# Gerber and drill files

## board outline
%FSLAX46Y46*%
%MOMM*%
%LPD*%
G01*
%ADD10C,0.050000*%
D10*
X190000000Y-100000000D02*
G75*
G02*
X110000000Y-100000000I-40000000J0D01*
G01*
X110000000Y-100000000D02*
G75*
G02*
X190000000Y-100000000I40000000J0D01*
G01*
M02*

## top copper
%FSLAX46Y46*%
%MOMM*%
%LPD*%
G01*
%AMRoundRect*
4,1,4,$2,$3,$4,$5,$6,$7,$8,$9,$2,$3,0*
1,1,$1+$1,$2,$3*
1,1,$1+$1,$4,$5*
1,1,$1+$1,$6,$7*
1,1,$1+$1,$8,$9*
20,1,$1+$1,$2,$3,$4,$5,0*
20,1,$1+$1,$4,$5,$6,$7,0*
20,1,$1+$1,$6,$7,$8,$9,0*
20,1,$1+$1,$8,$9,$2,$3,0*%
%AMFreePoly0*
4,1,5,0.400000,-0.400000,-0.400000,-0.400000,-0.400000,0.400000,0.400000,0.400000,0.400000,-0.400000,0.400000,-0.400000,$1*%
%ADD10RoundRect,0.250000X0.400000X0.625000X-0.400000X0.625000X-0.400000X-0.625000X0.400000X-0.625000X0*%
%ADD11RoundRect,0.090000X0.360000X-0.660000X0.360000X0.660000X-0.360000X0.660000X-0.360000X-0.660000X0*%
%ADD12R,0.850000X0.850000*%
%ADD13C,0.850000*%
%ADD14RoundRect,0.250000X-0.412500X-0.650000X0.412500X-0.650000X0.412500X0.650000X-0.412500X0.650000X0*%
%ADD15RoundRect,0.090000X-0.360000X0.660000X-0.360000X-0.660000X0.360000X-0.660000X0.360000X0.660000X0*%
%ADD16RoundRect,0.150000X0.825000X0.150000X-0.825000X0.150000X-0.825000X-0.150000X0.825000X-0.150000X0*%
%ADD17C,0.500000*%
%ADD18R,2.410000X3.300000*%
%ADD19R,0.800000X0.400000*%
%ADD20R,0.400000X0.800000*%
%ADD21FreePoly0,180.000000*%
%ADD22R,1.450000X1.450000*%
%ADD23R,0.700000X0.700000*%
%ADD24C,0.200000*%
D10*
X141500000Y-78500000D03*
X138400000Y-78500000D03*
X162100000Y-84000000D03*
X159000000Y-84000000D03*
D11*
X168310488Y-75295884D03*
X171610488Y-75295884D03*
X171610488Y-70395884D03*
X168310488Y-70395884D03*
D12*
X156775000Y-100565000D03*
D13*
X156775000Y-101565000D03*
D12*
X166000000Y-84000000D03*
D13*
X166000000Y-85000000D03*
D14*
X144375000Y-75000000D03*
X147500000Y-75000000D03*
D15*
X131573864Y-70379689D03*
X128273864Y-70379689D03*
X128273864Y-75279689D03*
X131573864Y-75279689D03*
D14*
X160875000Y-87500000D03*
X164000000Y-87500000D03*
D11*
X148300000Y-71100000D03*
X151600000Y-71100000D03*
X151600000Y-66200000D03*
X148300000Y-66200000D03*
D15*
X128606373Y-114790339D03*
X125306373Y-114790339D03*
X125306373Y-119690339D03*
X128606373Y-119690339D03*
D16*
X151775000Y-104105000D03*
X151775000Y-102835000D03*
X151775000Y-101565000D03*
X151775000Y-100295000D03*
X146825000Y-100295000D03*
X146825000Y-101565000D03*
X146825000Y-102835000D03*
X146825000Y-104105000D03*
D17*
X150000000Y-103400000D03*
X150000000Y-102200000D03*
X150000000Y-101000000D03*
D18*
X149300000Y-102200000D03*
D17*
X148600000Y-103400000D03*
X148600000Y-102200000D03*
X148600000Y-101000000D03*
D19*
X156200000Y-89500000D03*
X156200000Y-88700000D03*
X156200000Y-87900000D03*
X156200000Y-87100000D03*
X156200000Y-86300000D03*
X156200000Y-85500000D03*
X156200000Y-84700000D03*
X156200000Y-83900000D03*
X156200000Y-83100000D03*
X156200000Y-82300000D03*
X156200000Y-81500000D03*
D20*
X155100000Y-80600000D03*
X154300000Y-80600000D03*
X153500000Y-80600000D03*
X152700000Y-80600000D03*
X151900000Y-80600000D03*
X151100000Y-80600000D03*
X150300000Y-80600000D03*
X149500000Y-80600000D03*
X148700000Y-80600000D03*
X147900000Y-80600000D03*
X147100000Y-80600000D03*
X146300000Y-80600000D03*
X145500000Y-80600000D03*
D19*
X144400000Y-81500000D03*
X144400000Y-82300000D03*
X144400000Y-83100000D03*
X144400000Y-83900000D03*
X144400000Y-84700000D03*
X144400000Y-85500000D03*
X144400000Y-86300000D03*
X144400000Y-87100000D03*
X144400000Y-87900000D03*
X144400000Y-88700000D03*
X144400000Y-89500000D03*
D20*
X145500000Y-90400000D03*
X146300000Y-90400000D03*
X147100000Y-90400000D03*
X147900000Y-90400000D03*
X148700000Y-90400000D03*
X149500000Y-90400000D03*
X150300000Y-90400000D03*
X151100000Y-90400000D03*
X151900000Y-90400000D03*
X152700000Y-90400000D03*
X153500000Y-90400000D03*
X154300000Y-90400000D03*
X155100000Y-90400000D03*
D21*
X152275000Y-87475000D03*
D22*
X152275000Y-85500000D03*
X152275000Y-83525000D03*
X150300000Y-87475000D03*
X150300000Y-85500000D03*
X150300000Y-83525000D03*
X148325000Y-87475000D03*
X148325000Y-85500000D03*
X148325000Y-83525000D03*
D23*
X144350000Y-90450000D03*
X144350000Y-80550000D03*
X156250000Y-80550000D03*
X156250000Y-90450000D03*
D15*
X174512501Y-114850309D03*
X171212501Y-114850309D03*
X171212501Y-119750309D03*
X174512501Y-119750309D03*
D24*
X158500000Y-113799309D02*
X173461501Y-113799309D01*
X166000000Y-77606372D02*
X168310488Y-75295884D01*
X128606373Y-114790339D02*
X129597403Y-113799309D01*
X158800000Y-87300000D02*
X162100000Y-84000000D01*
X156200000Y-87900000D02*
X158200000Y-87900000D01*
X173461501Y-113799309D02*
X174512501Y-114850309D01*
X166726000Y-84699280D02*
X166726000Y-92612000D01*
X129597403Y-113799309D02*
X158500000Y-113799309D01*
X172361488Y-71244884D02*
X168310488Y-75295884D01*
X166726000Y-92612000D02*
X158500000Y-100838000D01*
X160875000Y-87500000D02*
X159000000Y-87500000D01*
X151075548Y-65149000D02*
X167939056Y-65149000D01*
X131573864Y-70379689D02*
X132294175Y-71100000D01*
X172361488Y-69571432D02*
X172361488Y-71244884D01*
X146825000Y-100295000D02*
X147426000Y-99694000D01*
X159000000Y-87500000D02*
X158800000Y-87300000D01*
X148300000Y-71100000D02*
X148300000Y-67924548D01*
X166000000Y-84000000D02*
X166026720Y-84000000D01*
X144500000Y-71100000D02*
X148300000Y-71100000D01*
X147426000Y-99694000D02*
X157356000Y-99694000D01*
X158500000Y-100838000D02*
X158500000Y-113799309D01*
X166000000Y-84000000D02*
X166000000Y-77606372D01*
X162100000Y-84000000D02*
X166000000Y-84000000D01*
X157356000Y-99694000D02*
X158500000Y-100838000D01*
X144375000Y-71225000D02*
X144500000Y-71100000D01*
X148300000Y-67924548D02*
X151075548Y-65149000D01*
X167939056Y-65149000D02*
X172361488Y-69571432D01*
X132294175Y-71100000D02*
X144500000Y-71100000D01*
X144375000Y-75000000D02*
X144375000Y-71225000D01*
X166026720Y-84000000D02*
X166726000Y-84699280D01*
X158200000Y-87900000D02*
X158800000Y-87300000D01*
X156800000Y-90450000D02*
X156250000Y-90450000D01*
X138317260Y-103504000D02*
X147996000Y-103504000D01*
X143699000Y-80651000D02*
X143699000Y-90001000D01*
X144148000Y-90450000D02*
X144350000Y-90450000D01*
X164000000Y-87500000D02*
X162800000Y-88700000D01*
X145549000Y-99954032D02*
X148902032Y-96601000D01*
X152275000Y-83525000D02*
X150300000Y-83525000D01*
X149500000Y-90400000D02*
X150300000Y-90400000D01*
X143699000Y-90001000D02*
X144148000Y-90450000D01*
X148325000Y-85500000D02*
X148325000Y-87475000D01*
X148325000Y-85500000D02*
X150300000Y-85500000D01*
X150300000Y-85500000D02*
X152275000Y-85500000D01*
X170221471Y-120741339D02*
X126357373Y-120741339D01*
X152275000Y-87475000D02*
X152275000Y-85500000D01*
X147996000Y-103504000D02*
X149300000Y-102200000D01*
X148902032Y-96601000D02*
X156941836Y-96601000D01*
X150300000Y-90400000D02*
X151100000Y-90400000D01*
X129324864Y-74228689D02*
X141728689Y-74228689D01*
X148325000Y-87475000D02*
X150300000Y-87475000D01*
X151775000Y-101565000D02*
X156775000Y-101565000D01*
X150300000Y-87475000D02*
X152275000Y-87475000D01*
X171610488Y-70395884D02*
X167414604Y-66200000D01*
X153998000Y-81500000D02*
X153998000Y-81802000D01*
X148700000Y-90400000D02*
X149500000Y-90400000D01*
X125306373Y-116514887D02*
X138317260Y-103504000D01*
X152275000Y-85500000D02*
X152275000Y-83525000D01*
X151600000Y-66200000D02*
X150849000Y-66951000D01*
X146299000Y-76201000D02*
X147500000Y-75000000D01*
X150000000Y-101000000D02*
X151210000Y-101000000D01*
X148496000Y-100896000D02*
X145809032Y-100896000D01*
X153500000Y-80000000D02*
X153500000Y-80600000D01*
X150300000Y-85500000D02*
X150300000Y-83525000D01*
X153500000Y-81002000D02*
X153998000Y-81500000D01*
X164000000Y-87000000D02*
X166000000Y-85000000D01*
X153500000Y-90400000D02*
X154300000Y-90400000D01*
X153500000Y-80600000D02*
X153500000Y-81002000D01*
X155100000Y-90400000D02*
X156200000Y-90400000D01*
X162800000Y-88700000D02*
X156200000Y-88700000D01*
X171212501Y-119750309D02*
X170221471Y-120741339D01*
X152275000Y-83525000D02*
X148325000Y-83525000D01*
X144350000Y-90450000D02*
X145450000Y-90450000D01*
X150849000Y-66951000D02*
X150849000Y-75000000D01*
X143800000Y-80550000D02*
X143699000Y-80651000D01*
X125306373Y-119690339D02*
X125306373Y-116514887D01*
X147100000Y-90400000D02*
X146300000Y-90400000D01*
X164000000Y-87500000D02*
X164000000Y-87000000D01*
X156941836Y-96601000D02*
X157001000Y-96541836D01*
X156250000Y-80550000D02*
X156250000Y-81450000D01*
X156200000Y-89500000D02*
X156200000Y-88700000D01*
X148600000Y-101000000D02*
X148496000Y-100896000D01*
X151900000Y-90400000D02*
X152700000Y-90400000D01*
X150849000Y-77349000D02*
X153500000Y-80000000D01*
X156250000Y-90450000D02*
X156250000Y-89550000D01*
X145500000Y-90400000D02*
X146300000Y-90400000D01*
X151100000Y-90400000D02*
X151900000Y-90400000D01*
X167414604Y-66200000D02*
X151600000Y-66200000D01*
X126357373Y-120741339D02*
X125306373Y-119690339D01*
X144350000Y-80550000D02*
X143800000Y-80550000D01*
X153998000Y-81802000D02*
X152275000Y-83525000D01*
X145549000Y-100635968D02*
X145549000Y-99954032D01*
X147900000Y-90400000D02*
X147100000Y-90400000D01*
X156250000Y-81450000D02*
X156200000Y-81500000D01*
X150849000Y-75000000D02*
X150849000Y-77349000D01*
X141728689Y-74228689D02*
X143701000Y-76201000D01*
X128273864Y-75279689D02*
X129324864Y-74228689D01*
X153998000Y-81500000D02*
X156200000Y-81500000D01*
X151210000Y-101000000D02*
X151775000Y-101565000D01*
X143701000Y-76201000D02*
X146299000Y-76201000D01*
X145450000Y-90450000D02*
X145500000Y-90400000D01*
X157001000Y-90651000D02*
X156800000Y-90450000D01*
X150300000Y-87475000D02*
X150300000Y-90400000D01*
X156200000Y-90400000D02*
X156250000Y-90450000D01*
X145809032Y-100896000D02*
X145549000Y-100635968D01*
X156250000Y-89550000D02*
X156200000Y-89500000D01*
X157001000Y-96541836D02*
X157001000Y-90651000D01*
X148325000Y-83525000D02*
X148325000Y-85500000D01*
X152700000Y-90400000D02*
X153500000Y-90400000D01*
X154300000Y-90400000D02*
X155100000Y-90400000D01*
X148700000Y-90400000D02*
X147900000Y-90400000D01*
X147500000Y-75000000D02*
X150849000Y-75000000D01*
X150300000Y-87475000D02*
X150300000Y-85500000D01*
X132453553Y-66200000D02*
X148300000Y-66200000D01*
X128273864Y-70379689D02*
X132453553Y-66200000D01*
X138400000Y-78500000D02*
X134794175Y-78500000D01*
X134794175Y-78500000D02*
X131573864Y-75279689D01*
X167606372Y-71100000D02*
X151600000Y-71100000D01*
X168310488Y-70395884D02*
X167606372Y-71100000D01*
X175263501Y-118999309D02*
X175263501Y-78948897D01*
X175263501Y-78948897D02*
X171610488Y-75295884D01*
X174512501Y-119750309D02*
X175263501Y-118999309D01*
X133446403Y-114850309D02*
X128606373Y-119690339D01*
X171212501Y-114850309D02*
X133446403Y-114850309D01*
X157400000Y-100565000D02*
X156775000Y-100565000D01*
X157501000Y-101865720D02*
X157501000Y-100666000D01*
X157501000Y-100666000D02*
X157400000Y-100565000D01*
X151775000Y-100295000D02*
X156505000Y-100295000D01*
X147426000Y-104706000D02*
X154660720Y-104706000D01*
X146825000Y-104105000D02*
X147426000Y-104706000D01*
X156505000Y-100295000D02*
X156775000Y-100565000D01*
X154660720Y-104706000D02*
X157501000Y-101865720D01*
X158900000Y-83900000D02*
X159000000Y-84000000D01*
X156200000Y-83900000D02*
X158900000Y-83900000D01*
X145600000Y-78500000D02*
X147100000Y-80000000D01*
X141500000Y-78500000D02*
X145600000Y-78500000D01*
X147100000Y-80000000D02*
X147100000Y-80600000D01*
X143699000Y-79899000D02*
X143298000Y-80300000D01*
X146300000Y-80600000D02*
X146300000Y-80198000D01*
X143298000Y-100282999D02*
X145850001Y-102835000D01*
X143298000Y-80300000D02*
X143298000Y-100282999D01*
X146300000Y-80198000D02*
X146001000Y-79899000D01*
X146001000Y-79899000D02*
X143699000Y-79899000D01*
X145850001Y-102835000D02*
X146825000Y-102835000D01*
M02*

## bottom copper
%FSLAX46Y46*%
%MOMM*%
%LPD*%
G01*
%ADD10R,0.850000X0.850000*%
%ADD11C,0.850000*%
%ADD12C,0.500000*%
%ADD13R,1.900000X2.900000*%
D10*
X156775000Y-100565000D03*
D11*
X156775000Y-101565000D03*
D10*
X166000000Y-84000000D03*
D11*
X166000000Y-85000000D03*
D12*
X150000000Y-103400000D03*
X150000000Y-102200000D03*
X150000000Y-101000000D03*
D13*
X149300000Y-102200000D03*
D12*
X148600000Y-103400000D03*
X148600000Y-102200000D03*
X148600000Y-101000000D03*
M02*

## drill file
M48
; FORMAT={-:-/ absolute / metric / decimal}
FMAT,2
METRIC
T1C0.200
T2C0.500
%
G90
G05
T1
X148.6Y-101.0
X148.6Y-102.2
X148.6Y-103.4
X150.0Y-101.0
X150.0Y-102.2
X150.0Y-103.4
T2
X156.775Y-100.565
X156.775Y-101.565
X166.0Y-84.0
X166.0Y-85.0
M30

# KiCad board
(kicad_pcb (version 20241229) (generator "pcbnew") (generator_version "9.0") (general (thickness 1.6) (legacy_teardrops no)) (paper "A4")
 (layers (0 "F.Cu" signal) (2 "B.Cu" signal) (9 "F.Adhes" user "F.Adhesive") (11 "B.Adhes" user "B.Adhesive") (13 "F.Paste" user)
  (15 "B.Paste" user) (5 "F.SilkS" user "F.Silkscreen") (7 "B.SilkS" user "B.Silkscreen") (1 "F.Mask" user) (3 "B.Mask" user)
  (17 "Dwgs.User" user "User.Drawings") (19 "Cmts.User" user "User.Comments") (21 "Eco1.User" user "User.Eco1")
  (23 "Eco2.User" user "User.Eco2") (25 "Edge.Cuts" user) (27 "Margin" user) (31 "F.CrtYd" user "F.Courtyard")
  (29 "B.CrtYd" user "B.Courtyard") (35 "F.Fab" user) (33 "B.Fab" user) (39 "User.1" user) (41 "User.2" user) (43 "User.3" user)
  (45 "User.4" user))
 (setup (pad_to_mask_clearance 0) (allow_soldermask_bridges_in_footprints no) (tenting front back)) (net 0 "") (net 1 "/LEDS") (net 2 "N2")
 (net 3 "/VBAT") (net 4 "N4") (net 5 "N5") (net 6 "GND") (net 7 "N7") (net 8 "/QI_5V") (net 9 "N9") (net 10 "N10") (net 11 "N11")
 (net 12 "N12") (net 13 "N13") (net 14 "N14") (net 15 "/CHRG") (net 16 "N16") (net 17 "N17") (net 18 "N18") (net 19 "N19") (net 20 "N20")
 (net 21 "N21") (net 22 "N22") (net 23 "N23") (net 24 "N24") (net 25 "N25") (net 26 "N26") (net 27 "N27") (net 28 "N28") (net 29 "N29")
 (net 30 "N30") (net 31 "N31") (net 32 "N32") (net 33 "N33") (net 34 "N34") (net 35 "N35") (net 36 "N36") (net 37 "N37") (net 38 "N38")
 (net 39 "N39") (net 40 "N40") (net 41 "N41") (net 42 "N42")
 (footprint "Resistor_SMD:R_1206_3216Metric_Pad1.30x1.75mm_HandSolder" (layer "F.Cu") (at 139.95 78.5 180)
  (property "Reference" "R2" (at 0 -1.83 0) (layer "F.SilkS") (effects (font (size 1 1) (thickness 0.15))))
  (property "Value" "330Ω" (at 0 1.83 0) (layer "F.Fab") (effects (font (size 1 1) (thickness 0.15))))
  (pad "1" smd roundrect (at -1.55 0 180) (size 1.3 1.75) (layers "F.Cu" "F.Mask" "F.Paste") (roundrect_rratio 0.192308) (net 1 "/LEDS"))
  (pad "2" smd roundrect (at 1.55 0 180) (size 1.3 1.75) (layers "F.Cu" "F.Mask" "F.Paste") (roundrect_rratio 0.192308) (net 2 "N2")))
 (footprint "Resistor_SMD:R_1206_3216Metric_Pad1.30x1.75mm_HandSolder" (layer "F.Cu") (at 160.55 84 180)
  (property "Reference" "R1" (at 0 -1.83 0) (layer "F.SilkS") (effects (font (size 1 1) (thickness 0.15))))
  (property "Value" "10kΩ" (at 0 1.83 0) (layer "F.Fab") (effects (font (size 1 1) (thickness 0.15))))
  (pad "1" smd roundrect (at -1.55 0 180) (size 1.3 1.75) (layers "F.Cu" "F.Mask" "F.Paste") (roundrect_rratio 0.192308) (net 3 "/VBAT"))
  (pad "2" smd roundrect (at 1.55 0 180) (size 1.3 1.75) (layers "F.Cu" "F.Mask" "F.Paste") (roundrect_rratio 0.192308) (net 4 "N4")))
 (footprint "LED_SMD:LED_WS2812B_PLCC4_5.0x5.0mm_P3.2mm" (layer "F.Cu") (at 169.960488 72.845884 90)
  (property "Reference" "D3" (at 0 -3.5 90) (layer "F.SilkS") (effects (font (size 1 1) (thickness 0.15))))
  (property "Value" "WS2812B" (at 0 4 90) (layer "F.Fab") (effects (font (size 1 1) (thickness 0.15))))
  (pad "1" smd roundrect (at -2.45 -1.65 90) (size 1.5 0.9) (layers "F.Cu" "F.Mask" "F.Paste") (roundrect_rratio 0.1) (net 3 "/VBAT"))
  (pad "2" smd roundrect (at -2.45 1.65 90) (size 1.5 0.9) (layers "F.Cu" "F.Mask" "F.Paste") (roundrect_rratio 0.1) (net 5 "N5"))
  (pad "3" smd roundrect (at 2.45 1.65 90) (size 1.5 0.9) (layers "F.Cu" "F.Mask" "F.Paste") (roundrect_rratio 0.1) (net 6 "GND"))
  (pad "4" smd roundrect (at 2.45 -1.65 90) (size 1.5 0.9) (layers "F.Cu" "F.Mask" "F.Paste") (roundrect_rratio 0.1) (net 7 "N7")))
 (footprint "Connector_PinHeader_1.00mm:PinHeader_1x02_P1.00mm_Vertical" (layer "F.Cu") (at 156.775 100.565)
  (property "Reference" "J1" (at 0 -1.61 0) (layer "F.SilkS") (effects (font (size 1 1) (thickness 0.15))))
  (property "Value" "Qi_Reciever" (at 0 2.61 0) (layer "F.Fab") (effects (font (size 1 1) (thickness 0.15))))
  (pad "1" thru_hole rect (at 0 0) (size 0.85 0.85) (drill 0.5) (layers "*.Cu" "*.Mask") (remove_unused_layers no) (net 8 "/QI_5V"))
  (pad "2" thru_hole circle (at 0 1) (size 0.85 0.85) (drill 0.5) (layers "*.Cu" "*.Mask") (remove_unused_layers no) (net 6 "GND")))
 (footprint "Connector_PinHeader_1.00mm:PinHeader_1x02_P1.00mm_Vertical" (layer "F.Cu") (at 166 84)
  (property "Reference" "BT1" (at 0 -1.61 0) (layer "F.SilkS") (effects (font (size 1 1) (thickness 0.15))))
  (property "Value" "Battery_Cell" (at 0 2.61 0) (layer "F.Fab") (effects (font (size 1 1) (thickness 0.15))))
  (pad "1" thru_hole rect (at 0 0) (size 0.85 0.85) (drill 0.5) (layers "*.Cu" "*.Mask") (remove_unused_layers no) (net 3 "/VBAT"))
  (pad "2" thru_hole circle (at 0 1) (size 0.85 0.85) (drill 0.5) (layers "*.Cu" "*.Mask") (remove_unused_layers no) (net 6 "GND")))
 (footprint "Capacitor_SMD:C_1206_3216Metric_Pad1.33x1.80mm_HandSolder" (layer "F.Cu") (at 145.9375 75)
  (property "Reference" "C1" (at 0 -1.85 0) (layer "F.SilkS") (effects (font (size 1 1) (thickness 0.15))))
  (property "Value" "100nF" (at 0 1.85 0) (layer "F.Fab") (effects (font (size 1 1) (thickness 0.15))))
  (pad "1" smd roundrect (at -1.5625 0) (size 1.325 1.8) (layers "F.Cu" "F.Mask" "F.Paste") (roundrect_rratio 0.188679) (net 3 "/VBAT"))
  (pad "2" smd roundrect (at 1.5625 0) (size 1.325 1.8) (layers "F.Cu" "F.Mask" "F.Paste") (roundrect_rratio 0.188679) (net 6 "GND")))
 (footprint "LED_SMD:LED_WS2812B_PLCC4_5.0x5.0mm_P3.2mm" (layer "F.Cu") (at 129.923864 72.829689 -90)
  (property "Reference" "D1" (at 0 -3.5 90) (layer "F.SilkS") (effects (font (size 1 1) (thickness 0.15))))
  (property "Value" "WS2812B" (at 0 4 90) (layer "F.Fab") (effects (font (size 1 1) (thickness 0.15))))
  (pad "1" smd roundrect (at -2.45 -1.65 270) (size 1.5 0.9) (layers "F.Cu" "F.Mask" "F.Paste") (roundrect_rratio 0.1) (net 3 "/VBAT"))
  (pad "2" smd roundrect (at -2.45 1.65 270) (size 1.5 0.9) (layers "F.Cu" "F.Mask" "F.Paste") (roundrect_rratio 0.1) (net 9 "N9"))
  (pad "3" smd roundrect (at 2.45 1.65 270) (size 1.5 0.9) (layers "F.Cu" "F.Mask" "F.Paste") (roundrect_rratio 0.1) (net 6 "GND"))
  (pad "4" smd roundrect (at 2.45 -1.65 270) (size 1.5 0.9) (layers "F.Cu" "F.Mask" "F.Paste") (roundrect_rratio 0.1) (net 2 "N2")))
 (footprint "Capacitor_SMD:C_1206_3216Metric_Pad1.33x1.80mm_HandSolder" (layer "F.Cu") (at 162.4375 87.5)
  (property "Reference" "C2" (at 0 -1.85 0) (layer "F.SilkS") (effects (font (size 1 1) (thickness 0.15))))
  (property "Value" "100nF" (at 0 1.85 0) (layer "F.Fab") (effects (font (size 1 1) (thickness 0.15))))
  (pad "1" smd roundrect (at -1.5625 0) (size 1.325 1.8) (layers "F.Cu" "F.Mask" "F.Paste") (roundrect_rratio 0.188679) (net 3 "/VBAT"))
  (pad "2" smd roundrect (at 1.5625 0) (size 1.325 1.8) (layers "F.Cu" "F.Mask" "F.Paste") (roundrect_rratio 0.188679) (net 6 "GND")))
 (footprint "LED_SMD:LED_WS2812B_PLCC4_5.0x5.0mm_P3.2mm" (layer "F.Cu") (at 149.95 68.65 90)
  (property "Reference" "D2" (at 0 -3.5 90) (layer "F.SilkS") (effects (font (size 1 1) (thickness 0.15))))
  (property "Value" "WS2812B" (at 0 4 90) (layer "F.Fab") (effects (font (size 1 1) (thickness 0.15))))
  (pad "1" smd roundrect (at -2.45 -1.65 90) (size 1.5 0.9) (layers "F.Cu" "F.Mask" "F.Paste") (roundrect_rratio 0.1) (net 3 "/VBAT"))
  (pad "2" smd roundrect (at -2.45 1.65 90) (size 1.5 0.9) (layers "F.Cu" "F.Mask" "F.Paste") (roundrect_rratio 0.1) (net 7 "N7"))
  (pad "3" smd roundrect (at 2.45 1.65 90) (size 1.5 0.9) (layers "F.Cu" "F.Mask" "F.Paste") (roundrect_rratio 0.1) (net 6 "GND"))
  (pad "4" smd roundrect (at 2.45 -1.65 90) (size 1.5 0.9) (layers "F.Cu" "F.Mask" "F.Paste") (roundrect_rratio 0.1) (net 9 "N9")))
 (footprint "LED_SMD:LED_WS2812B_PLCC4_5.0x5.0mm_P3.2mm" (layer "F.Cu") (at 126.956373 117.240339 -90)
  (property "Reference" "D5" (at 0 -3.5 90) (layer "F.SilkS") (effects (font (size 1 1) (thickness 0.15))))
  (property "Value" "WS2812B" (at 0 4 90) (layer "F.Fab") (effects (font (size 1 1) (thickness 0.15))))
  (pad "1" smd roundrect (at -2.45 -1.65 270) (size 1.5 0.9) (layers "F.Cu" "F.Mask" "F.Paste") (roundrect_rratio 0.1) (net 3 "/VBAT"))
  (pad "2" smd roundrect (at -2.45 1.65 270) (size 1.5 0.9) (layers "F.Cu" "F.Mask" "F.Paste") (roundrect_rratio 0.1) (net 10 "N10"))
  (pad "3" smd roundrect (at 2.45 1.65 270) (size 1.5 0.9) (layers "F.Cu" "F.Mask" "F.Paste") (roundrect_rratio 0.1) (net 6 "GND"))
  (pad "4" smd roundrect (at 2.45 -1.65 270) (size 1.5 0.9) (layers "F.Cu" "F.Mask" "F.Paste") (roundrect_rratio 0.1) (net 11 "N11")))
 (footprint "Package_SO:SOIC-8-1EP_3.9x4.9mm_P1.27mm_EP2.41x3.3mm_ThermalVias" (layer "F.Cu") (at 149.3 102.2 180)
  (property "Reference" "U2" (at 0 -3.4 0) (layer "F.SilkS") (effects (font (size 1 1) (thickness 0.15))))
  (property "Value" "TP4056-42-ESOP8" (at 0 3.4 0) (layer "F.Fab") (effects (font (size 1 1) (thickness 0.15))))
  (pad "" smd roundrect (at -0.6 -0.825 180) (size 1.01 1.38) (layers "F.Paste") (roundrect_rratio 0.247525))
  (pad "" smd roundrect (at -0.6 0.825 180) (size 1.01 1.38) (layers "F.Paste") (roundrect_rratio 0.247525))
  (pad "" smd roundrect (at 0.6 -0.825 180) (size 1.01 1.38) (layers "F.Paste") (roundrect_rratio 0.247525))
  (pad "" smd roundrect (at 0.6 0.825 180) (size 1.01 1.38) (layers "F.Paste") (roundrect_rratio 0.247525))
  (pad "1" smd roundrect (at -2.475 -1.905 180) (size 1.95 0.6) (layers "F.Cu" "F.Mask" "F.Paste") (roundrect_rratio 0.25) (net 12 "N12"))
  (pad "2" smd roundrect (at -2.475 -0.635 180) (size 1.95 0.6) (layers "F.Cu" "F.Mask" "F.Paste") (roundrect_rratio 0.25) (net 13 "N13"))
  (pad "3" smd roundrect (at -2.475 0.635 180) (size 1.95 0.6) (layers "F.Cu" "F.Mask" "F.Paste") (roundrect_rratio 0.25) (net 6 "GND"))
  (pad "4" smd roundrect (at -2.475 1.905 180) (size 1.95 0.6) (layers "F.Cu" "F.Mask" "F.Paste") (roundrect_rratio 0.25) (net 8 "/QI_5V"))
  (pad "5" smd roundrect (at 2.475 1.905 180) (size 1.95 0.6) (layers "F.Cu" "F.Mask" "F.Paste") (roundrect_rratio 0.25) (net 3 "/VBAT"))
  (pad "6" smd roundrect (at 2.475 0.635 180) (size 1.95 0.6) (layers "F.Cu" "F.Mask" "F.Paste") (roundrect_rratio 0.25) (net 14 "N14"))
  (pad "7" smd roundrect (at 2.475 -0.635 180) (size 1.95 0.6) (layers "F.Cu" "F.Mask" "F.Paste") (roundrect_rratio 0.25) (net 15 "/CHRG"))
  (pad "8" smd roundrect (at 2.475 -1.905 180) (size 1.95 0.6) (layers "F.Cu" "F.Mask" "F.Paste") (roundrect_rratio 0.25) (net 8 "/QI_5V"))
  (pad "9" thru_hole circle (at -0.7 -1.2 180) (size 0.5 0.5) (drill 0.2) (layers "*.Cu") (remove_unused_layers no) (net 6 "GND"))
  (pad "9" thru_hole circle (at -0.7 0 180) (size 0.5 0.5) (drill 0.2) (layers "*.Cu") (remove_unused_layers no) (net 6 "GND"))
  (pad "9" thru_hole circle (at -0.7 1.2 180) (size 0.5 0.5) (drill 0.2) (layers "*.Cu") (remove_unused_layers no) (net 6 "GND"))
  (pad "9" smd rect (at 0 0 180) (size 1.9 2.9) (layers "B.Cu") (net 6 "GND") (zone_connect 2))
  (pad "9" smd rect (at 0 0 180) (size 2.41 3.3) (layers "F.Cu" "F.Mask") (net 6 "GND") (zone_connect 2))
  (pad "9" thru_hole circle (at 0.7 -1.2 180) (size 0.5 0.5) (drill 0.2) (layers "*.Cu") (remove_unused_layers no) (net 6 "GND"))
  (pad "9" thru_hole circle (at 0.7 0 180) (size 0.5 0.5) (drill 0.2) (layers "*.Cu") (remove_unused_layers no) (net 6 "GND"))
  (pad "9" thru_hole circle (at 0.7 1.2 180) (size 0.5 0.5) (drill 0.2) (layers "*.Cu") (remove_unused_layers no) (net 6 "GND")))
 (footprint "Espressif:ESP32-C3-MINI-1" (layer "F.Cu") (at 150.3 88.2 180)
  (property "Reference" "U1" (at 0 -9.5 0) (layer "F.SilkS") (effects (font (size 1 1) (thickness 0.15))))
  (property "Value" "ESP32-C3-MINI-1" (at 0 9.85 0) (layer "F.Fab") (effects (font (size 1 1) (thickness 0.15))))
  (pad "1" smd rect (at -5.9 -1.3 270) (size 0.4 0.8) (layers "F.Cu" "F.Mask" "F.Paste") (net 6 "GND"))
  (pad "2" smd rect (at -5.9 -0.5 270) (size 0.4 0.8) (layers "F.Cu" "F.Mask" "F.Paste") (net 6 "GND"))
  (pad "3" smd rect (at -5.9 0.3 270) (size 0.4 0.8) (layers "F.Cu" "F.Mask" "F.Paste") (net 3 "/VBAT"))
  (pad "4" smd rect (at -5.9 1.1 270) (size 0.4 0.8) (layers "F.Cu" "F.Mask" "F.Paste") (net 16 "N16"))
  (pad "5" smd rect (at -5.9 1.9 270) (size 0.4 0.8) (layers "F.Cu" "F.Mask" "F.Paste") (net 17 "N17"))
  (pad "6" smd rect (at -5.9 2.7 270) (size 0.4 0.8) (layers "F.Cu" "F.Mask" "F.Paste") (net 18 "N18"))
  (pad "7" smd rect (at -5.9 3.5 270) (size 0.4 0.8) (layers "F.Cu" "F.Mask" "F.Paste") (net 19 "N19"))
  (pad "8" smd rect (at -5.9 4.3 270) (size 0.4 0.8) (layers "F.Cu" "F.Mask" "F.Paste") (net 4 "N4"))
  (pad "9" smd rect (at -5.9 5.1 270) (size 0.4 0.8) (layers "F.Cu" "F.Mask" "F.Paste") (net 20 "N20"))
  (pad "10" smd rect (at -5.9 5.9 270) (size 0.4 0.8) (layers "F.Cu" "F.Mask" "F.Paste") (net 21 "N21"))
  (pad "11" smd rect (at -5.9 6.7 270) (size 0.4 0.8) (layers "F.Cu" "F.Mask" "F.Paste") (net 6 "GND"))
  (pad "12" smd rect (at -4.8 7.6 180) (size 0.4 0.8) (layers "F.Cu" "F.Mask" "F.Paste") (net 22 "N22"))
  (pad "13" smd rect (at -4 7.6 180) (size 0.4 0.8) (layers "F.Cu" "F.Mask" "F.Paste") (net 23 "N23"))
  (pad "14" smd rect (at -3.2 7.6 180) (size 0.4 0.8) (layers "F.Cu" "F.Mask" "F.Paste") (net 6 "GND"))
  (pad "15" smd rect (at -2.4 7.6 180) (size 0.4 0.8) (layers "F.Cu" "F.Mask" "F.Paste") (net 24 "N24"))
  (pad "16" smd rect (at -1.6 7.6 180) (size 0.4 0.8) (layers "F.Cu" "F.Mask" "F.Paste") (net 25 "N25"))
  (pad "17" smd rect (at -0.8 7.6 180) (size 0.4 0.8) (layers "F.Cu" "F.Mask" "F.Paste") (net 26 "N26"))
  (pad "18" smd rect (at 0 7.6 180) (size 0.4 0.8) (layers "F.Cu" "F.Mask" "F.Paste") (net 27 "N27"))
  (pad "19" smd rect (at 0.8 7.6 180) (size 0.4 0.8) (layers "F.Cu" "F.Mask" "F.Paste") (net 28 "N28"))
  (pad "20" smd rect (at 1.6 7.6 180) (size 0.4 0.8) (layers "F.Cu" "F.Mask" "F.Paste") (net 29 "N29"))
  (pad "21" smd rect (at 2.4 7.6 180) (size 0.4 0.8) (layers "F.Cu" "F.Mask" "F.Paste") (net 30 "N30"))
  (pad "22" smd rect (at 3.2 7.6 180) (size 0.4 0.8) (layers "F.Cu" "F.Mask" "F.Paste") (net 1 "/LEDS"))
  (pad "23" smd rect (at 4 7.6 180) (size 0.4 0.8) (layers "F.Cu" "F.Mask" "F.Paste") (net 15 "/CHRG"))
  (pad "24" smd rect (at 4.8 7.6 180) (size 0.4 0.8) (layers "F.Cu" "F.Mask" "F.Paste") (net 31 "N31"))
  (pad "25" smd rect (at 5.9 6.7 270) (size 0.4 0.8) (layers "F.Cu" "F.Mask" "F.Paste") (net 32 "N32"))
  (pad "26" smd rect (at 5.9 5.9 270) (size 0.4 0.8) (layers "F.Cu" "F.Mask" "F.Paste") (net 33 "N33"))
  (pad "27" smd rect (at 5.9 5.1 270) (size 0.4 0.8) (layers "F.Cu" "F.Mask" "F.Paste") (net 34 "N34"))
  (pad "28" smd rect (at 5.9 4.3 270) (size 0.4 0.8) (layers "F.Cu" "F.Mask" "F.Paste") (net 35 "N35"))
  (pad "29" smd rect (at 5.9 3.5 270) (size 0.4 0.8) (layers "F.Cu" "F.Mask" "F.Paste") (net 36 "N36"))
  (pad "30" smd rect (at 5.9 2.7 270) (size 0.4 0.8) (layers "F.Cu" "F.Mask" "F.Paste") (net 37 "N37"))
  (pad "31" smd rect (at 5.9 1.9 270) (size 0.4 0.8) (layers "F.Cu" "F.Mask" "F.Paste") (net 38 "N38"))
  (pad "32" smd rect (at 5.9 1.1 270) (size 0.4 0.8) (layers "F.Cu" "F.Mask" "F.Paste") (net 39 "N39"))
  (pad "33" smd rect (at 5.9 0.3 270) (size 0.4 0.8) (layers "F.Cu" "F.Mask" "F.Paste") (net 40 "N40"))
  (pad "34" smd rect (at 5.9 -0.5 270) (size 0.4 0.8) (layers "F.Cu" "F.Mask" "F.Paste") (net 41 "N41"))
  (pad "35" smd rect (at 5.9 -1.3 270) (size 0.4 0.8) (layers "F.Cu" "F.Mask" "F.Paste") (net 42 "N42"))
  (pad "36" smd rect (at 4.8 -2.2 180) (size 0.4 0.8) (layers "F.Cu" "F.Mask" "F.Paste") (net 6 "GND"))
  (pad "37" smd rect (at 4 -2.2 180) (size 0.4 0.8) (layers "F.Cu" "F.Mask" "F.Paste") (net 6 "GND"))
  (pad "38" smd rect (at 3.2 -2.2 180) (size 0.4 0.8) (layers "F.Cu" "F.Mask" "F.Paste") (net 6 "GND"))
  (pad "39" smd rect (at 2.4 -2.2 180) (size 0.4 0.8) (layers "F.Cu" "F.Mask" "F.Paste") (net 6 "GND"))
  (pad "40" smd rect (at 1.6 -2.2 180) (size 0.4 0.8) (layers "F.Cu" "F.Mask" "F.Paste") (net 6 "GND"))
  (pad "41" smd rect (at 0.8 -2.2 180) (size 0.4 0.8) (layers "F.Cu" "F.Mask" "F.Paste") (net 6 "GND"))
  (pad "42" smd rect (at 0 -2.2 180) (size 0.4 0.8) (layers "F.Cu" "F.Mask" "F.Paste") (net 6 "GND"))
  (pad "43" smd rect (at -0.8 -2.2 180) (size 0.4 0.8) (layers "F.Cu" "F.Mask" "F.Paste") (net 6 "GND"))
  (pad "44" smd rect (at -1.6 -2.2 180) (size 0.4 0.8) (layers "F.Cu" "F.Mask" "F.Paste") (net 6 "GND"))
  (pad "45" smd rect (at -2.4 -2.2 180) (size 0.4 0.8) (layers "F.Cu" "F.Mask" "F.Paste") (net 6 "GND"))
  (pad "46" smd rect (at -3.2 -2.2 180) (size 0.4 0.8) (layers "F.Cu" "F.Mask" "F.Paste") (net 6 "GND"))
  (pad "47" smd rect (at -4 -2.2 180) (size 0.4 0.8) (layers "F.Cu" "F.Mask" "F.Paste") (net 6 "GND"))
  (pad "48" smd rect (at -4.8 -2.2 180) (size 0.4 0.8) (layers "F.Cu" "F.Mask" "F.Paste") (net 6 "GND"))
  (pad "49" smd custom (at -1.975 0.725 180) (size 0.8 0.8) (layers "F.Cu" "F.Mask" "F.Paste") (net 6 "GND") (zone_connect 2)
   (thermal_bridge_angle 45) (options (clearance outline) (anchor rect)) (primitives))
  (pad "49" smd rect (at -1.975 2.7 270) (size 1.45 1.45) (layers "F.Cu" "F.Mask" "F.Paste") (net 6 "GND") (zone_connect 2))
  (pad "49" smd rect (at -1.975 4.675 270) (size 1.45 1.45) (layers "F.Cu" "F.Mask" "F.Paste") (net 6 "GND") (zone_connect 2))
  (pad "49" smd rect (at 0 0.725 270) (size 1.45 1.45) (layers "F.Cu" "F.Mask" "F.Paste") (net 6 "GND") (zone_connect 2))
  (pad "49" smd rect (at 0 2.7 270) (size 1.45 1.45) (layers "F.Cu" "F.Mask" "F.Paste") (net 6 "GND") (zone_connect 2))
  (pad "49" smd rect (at 0 4.675 270) (size 1.45 1.45) (layers "F.Cu" "F.Mask" "F.Paste") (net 6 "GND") (zone_connect 2))
  (pad "49" smd rect (at 1.975 0.725 270) (size 1.45 1.45) (layers "F.Cu" "F.Mask" "F.Paste") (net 6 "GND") (zone_connect 2))
  (pad "49" smd rect (at 1.975 2.7 270) (size 1.45 1.45) (layers "F.Cu" "F.Mask" "F.Paste") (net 6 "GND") (zone_connect 2))
  (pad "49" smd rect (at 1.975 4.675 270) (size 1.45 1.45) (layers "F.Cu" "F.Mask" "F.Paste") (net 6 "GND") (zone_connect 2))
  (pad "50" smd rect (at 5.95 -2.25 270) (size 0.7 0.7) (layers "F.Cu" "F.Mask" "F.Paste") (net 6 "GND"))
  (pad "51" smd rect (at 5.95 7.65 270) (size 0.7 0.7) (layers "F.Cu" "F.Mask" "F.Paste") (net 6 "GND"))
  (pad "52" smd rect (at -5.95 7.65 270) (size 0.7 0.7) (layers "F.Cu" "F.Mask" "F.Paste") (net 6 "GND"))
  (pad "53" smd rect (at -5.95 -2.25 270) (size 0.7 0.7) (layers "F.Cu" "F.Mask" "F.Paste") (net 6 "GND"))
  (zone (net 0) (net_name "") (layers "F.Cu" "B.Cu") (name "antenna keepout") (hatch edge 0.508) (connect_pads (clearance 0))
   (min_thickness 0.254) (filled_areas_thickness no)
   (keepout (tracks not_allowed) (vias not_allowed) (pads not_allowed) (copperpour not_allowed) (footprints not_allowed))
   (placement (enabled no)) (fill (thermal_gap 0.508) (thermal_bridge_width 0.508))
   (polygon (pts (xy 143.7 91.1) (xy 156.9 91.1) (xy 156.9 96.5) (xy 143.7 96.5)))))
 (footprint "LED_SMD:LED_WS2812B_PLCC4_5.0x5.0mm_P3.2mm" (layer "F.Cu") (at 172.862501 117.300309 -90)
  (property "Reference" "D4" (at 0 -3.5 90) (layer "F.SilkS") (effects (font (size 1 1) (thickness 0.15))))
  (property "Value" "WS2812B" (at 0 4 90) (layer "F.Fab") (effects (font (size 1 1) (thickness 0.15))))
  (pad "1" smd roundrect (at -2.45 -1.65 270) (size 1.5 0.9) (layers "F.Cu" "F.Mask" "F.Paste") (roundrect_rratio 0.1) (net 3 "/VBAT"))
  (pad "2" smd roundrect (at -2.45 1.65 270) (size 1.5 0.9) (layers "F.Cu" "F.Mask" "F.Paste") (roundrect_rratio 0.1) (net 11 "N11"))
  (pad "3" smd roundrect (at 2.45 1.65 270) (size 1.5 0.9) (layers "F.Cu" "F.Mask" "F.Paste") (roundrect_rratio 0.1) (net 6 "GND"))
  (pad "4" smd roundrect (at 2.45 -1.65 270) (size 1.5 0.9) (layers "F.Cu" "F.Mask" "F.Paste") (roundrect_rratio 0.1) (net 5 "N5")))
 (gr_circle (center 150 100) (end 190 100) (stroke (width 0.05) (type default)) (fill no) (layer "Edge.Cuts"))
 (segment (start 158.5 113.799309) (end 173.461501 113.799309) (width 0.2) (layer "F.Cu") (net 3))
 (segment (start 166 77.606372) (end 168.310488 75.295884) (width 0.2) (layer "F.Cu") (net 3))
 (segment (start 128.606373 114.790339) (end 129.597403 113.799309) (width 0.2) (layer "F.Cu") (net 3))
 (segment (start 158.8 87.3) (end 162.1 84) (width 0.2) (layer "F.Cu") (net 3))
 (segment (start 156.2 87.9) (end 158.2 87.9) (width 0.2) (layer "F.Cu") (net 3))
 (segment (start 173.461501 113.799309) (end 174.512501 114.850309) (width 0.2) (layer "F.Cu") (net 3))
 (segment (start 166.726 84.69928) (end 166.726 92.612) (width 0.2) (layer "F.Cu") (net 3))
 (segment (start 129.597403 113.799309) (end 158.5 113.799309) (width 0.2) (layer "F.Cu") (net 3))
 (segment (start 172.361488 71.244884) (end 168.310488 75.295884) (width 0.2) (layer "F.Cu") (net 3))
 (segment (start 166.726 92.612) (end 158.5 100.838) (width 0.2) (layer "F.Cu") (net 3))
 (segment (start 160.875 87.5) (end 159 87.5) (width 0.2) (layer "F.Cu") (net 3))
 (segment (start 151.075548 65.149) (end 167.939056 65.149) (width 0.2) (layer "F.Cu") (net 3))
 (segment (start 131.573864 70.379689) (end 132.294175 71.1) (width 0.2) (layer "F.Cu") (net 3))
 (segment (start 172.361488 69.571432) (end 172.361488 71.244884) (width 0.2) (layer "F.Cu") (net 3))
 (segment (start 146.825 100.295) (end 147.426 99.694) (width 0.2) (layer "F.Cu") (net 3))
 (segment (start 159 87.5) (end 158.8 87.3) (width 0.2) (layer "F.Cu") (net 3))
 (segment (start 148.3 71.1) (end 148.3 67.924548) (width 0.2) (layer "F.Cu") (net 3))
 (segment (start 166 84) (end 166.02672 84) (width 0.2) (layer "F.Cu") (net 3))
 (segment (start 144.5 71.1) (end 148.3 71.1) (width 0.2) (layer "F.Cu") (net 3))
 (segment (start 147.426 99.694) (end 157.356 99.694) (width 0.2) (layer "F.Cu") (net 3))
 (segment (start 158.5 100.838) (end 158.5 113.799309) (width 0.2) (layer "F.Cu") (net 3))
 (segment (start 166 84) (end 166 77.606372) (width 0.2) (layer "F.Cu") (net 3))
 (segment (start 162.1 84) (end 166 84) (width 0.2) (layer "F.Cu") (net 3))
 (segment (start 157.356 99.694) (end 158.5 100.838) (width 0.2) (layer "F.Cu") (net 3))
 (segment (start 144.375 71.225) (end 144.5 71.1) (width 0.2) (layer "F.Cu") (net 3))
 (segment (start 148.3 67.924548) (end 151.075548 65.149) (width 0.2) (layer "F.Cu") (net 3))
 (segment (start 167.939056 65.149) (end 172.361488 69.571432) (width 0.2) (layer "F.Cu") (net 3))
 (segment (start 132.294175 71.1) (end 144.5 71.1) (width 0.2) (layer "F.Cu") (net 3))
 (segment (start 144.375 75) (end 144.375 71.225) (width 0.2) (layer "F.Cu") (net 3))
 (segment (start 166.02672 84) (end 166.726 84.69928) (width 0.2) (layer "F.Cu") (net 3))
 (segment (start 158.2 87.9) (end 158.8 87.3) (width 0.2) (layer "F.Cu") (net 3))
 (segment (start 156.8 90.45) (end 156.25 90.45) (width 0.2) (layer "F.Cu") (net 6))
 (segment (start 138.31726 103.504) (end 147.996 103.504) (width 0.2) (layer "F.Cu") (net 6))
 (segment (start 143.699 80.651) (end 143.699 90.001) (width 0.2) (layer "F.Cu") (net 6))
 (segment (start 144.148 90.45) (end 144.35 90.45) (width 0.2) (layer "F.Cu") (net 6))
 (segment (start 164 87.5) (end 162.8 88.7) (width 0.2) (layer "F.Cu") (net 6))
 (segment (start 145.549 99.954032) (end 148.902032 96.601) (width 0.2) (layer "F.Cu") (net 6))
 (segment (start 152.275 83.525) (end 150.3 83.525) (width 0.2) (layer "F.Cu") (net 6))
 (segment (start 149.5 90.4) (end 150.3 90.4) (width 0.2) (layer "F.Cu") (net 6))
 (segment (start 143.699 90.001) (end 144.148 90.45) (width 0.2) (layer "F.Cu") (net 6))
 (segment (start 148.325 85.5) (end 148.325 87.475) (width 0.2) (layer "F.Cu") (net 6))
 (segment (start 148.325 85.5) (end 150.3 85.5) (width 0.2) (layer "F.Cu") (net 6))
 (segment (start 150.3 85.5) (end 152.275 85.5) (width 0.2) (layer "F.Cu") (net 6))
 (segment (start 170.221471 120.741339) (end 126.357373 120.741339) (width 0.2) (layer "F.Cu") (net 6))
 (segment (start 152.275 87.475) (end 152.275 85.5) (width 0.2) (layer "F.Cu") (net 6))
 (segment (start 147.996 103.504) (end 149.3 102.2) (width 0.2) (layer "F.Cu") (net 6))
 (segment (start 148.902032 96.601) (end 156.941836 96.601) (width 0.2) (layer "F.Cu") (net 6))
 (segment (start 150.3 90.4) (end 151.1 90.4) (width 0.2) (layer "F.Cu") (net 6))
 (segment (start 129.324864 74.228689) (end 141.728689 74.228689) (width 0.2) (layer "F.Cu") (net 6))
 (segment (start 148.325 87.475) (end 150.3 87.475) (width 0.2) (layer "F.Cu") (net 6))
 (segment (start 151.775 101.565) (end 156.775 101.565) (width 0.2) (layer "F.Cu") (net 6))
 (segment (start 150.3 87.475) (end 152.275 87.475) (width 0.2) (layer "F.Cu") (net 6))
 (segment (start 171.610488 70.395884) (end 167.414604 66.2) (width 0.2) (layer "F.Cu") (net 6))
 (segment (start 153.998 81.5) (end 153.998 81.802) (width 0.2) (layer "F.Cu") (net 6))
 (segment (start 148.7 90.4) (end 149.5 90.4) (width 0.2) (layer "F.Cu") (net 6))
 (segment (start 125.306373 116.514887) (end 138.31726 103.504) (width 0.2) (layer "F.Cu") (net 6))
 (segment (start 152.275 85.5) (end 152.275 83.525) (width 0.2) (layer "F.Cu") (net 6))
 (segment (start 151.6 66.2) (end 150.849 66.951) (width 0.2) (layer "F.Cu") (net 6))
 (segment (start 146.299 76.201) (end 147.5 75) (width 0.2) (layer "F.Cu") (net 6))
 (segment (start 150 101) (end 151.21 101) (width 0.2) (layer "F.Cu") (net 6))
 (segment (start 148.496 100.896) (end 145.809032 100.896) (width 0.2) (layer "F.Cu") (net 6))
 (segment (start 153.5 80) (end 153.5 80.6) (width 0.2) (layer "F.Cu") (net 6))
 (segment (start 150.3 85.5) (end 150.3 83.525) (width 0.2) (layer "F.Cu") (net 6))
 (segment (start 153.5 81.002) (end 153.998 81.5) (width 0.2) (layer "F.Cu") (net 6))
 (segment (start 164 87) (end 166 85) (width 0.2) (layer "F.Cu") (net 6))
 (segment (start 153.5 90.4) (end 154.3 90.4) (width 0.2) (layer "F.Cu") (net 6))
 (segment (start 153.5 80.6) (end 153.5 81.002) (width 0.2) (layer "F.Cu") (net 6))
 (segment (start 155.1 90.4) (end 156.2 90.4) (width 0.2) (layer "F.Cu") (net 6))
 (segment (start 162.8 88.7) (end 156.2 88.7) (width 0.2) (layer "F.Cu") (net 6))
 (segment (start 171.212501 119.750309) (end 170.221471 120.741339) (width 0.2) (layer "F.Cu") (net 6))
 (segment (start 152.275 83.525) (end 148.325 83.525) (width 0.2) (layer "F.Cu") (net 6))
 (segment (start 144.35 90.45) (end 145.45 90.45) (width 0.2) (layer "F.Cu") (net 6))
 (segment (start 150.849 66.951) (end 150.849 75) (width 0.2) (layer "F.Cu") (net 6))
 (segment (start 143.8 80.55) (end 143.699 80.651) (width 0.2) (layer "F.Cu") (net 6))
 (segment (start 125.306373 119.690339) (end 125.306373 116.514887) (width 0.2) (layer "F.Cu") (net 6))
 (segment (start 147.1 90.4) (end 146.3 90.4) (width 0.2) (layer "F.Cu") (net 6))
 (segment (start 164 87.5) (end 164 87) (width 0.2) (layer "F.Cu") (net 6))
 (segment (start 156.941836 96.601) (end 157.001 96.541836) (width 0.2) (layer "F.Cu") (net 6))
 (segment (start 156.25 80.55) (end 156.25 81.45) (width 0.2) (layer "F.Cu") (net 6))
 (segment (start 156.2 89.5) (end 156.2 88.7) (width 0.2) (layer "F.Cu") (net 6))
 (segment (start 148.6 101) (end 148.496 100.896) (width 0.2) (layer "F.Cu") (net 6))
 (segment (start 151.9 90.4) (end 152.7 90.4) (width 0.2) (layer "F.Cu") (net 6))
 (segment (start 150.849 77.349) (end 153.5 80) (width 0.2) (layer "F.Cu") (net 6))
 (segment (start 156.25 90.45) (end 156.25 89.55) (width 0.2) (layer "F.Cu") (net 6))
 (segment (start 145.5 90.4) (end 146.3 90.4) (width 0.2) (layer "F.Cu") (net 6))
 (segment (start 151.1 90.4) (end 151.9 90.4) (width 0.2) (layer "F.Cu") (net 6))
 (segment (start 167.414604 66.2) (end 151.6 66.2) (width 0.2) (layer "F.Cu") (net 6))
 (segment (start 126.357373 120.741339) (end 125.306373 119.690339) (width 0.2) (layer "F.Cu") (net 6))
 (segment (start 144.35 80.55) (end 143.8 80.55) (width 0.2) (layer "F.Cu") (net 6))
 (segment (start 153.998 81.802) (end 152.275 83.525) (width 0.2) (layer "F.Cu") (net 6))
 (segment (start 145.549 100.635968) (end 145.549 99.954032) (width 0.2) (layer "F.Cu") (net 6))
 (segment (start 147.9 90.4) (end 147.1 90.4) (width 0.2) (layer "F.Cu") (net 6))
 (segment (start 156.25 81.45) (end 156.2 81.5) (width 0.2) (layer "F.Cu") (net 6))
 (segment (start 150.849 75) (end 150.849 77.349) (width 0.2) (layer "F.Cu") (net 6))
 (segment (start 141.728689 74.228689) (end 143.701 76.201) (width 0.2) (layer "F.Cu") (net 6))
 (segment (start 128.273864 75.279689) (end 129.324864 74.228689) (width 0.2) (layer "F.Cu") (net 6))
 (segment (start 153.998 81.5) (end 156.2 81.5) (width 0.2) (layer "F.Cu") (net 6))
 (segment (start 151.21 101) (end 151.775 101.565) (width 0.2) (layer "F.Cu") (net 6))
 (segment (start 143.701 76.201) (end 146.299 76.201) (width 0.2) (layer "F.Cu") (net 6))
 (segment (start 145.45 90.45) (end 145.5 90.4) (width 0.2) (layer "F.Cu") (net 6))
 (segment (start 157.001 90.651) (end 156.8 90.45) (width 0.2) (layer "F.Cu") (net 6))
 (segment (start 150.3 87.475) (end 150.3 90.4) (width 0.2) (layer "F.Cu") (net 6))
 (segment (start 156.2 90.4) (end 156.25 90.45) (width 0.2) (layer "F.Cu") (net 6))
 (segment (start 145.809032 100.896) (end 145.549 100.635968) (width 0.2) (layer "F.Cu") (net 6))
 (segment (start 156.25 89.55) (end 156.2 89.5) (width 0.2) (layer "F.Cu") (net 6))
 (segment (start 157.001 96.541836) (end 157.001 90.651) (width 0.2) (layer "F.Cu") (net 6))
 (segment (start 148.325 83.525) (end 148.325 85.5) (width 0.2) (layer "F.Cu") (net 6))
 (segment (start 152.7 90.4) (end 153.5 90.4) (width 0.2) (layer "F.Cu") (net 6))
 (segment (start 154.3 90.4) (end 155.1 90.4) (width 0.2) (layer "F.Cu") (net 6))
 (segment (start 148.7 90.4) (end 147.9 90.4) (width 0.2) (layer "F.Cu") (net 6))
 (segment (start 147.5 75) (end 150.849 75) (width 0.2) (layer "F.Cu") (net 6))
 (segment (start 150.3 87.475) (end 150.3 85.5) (width 0.2) (layer "F.Cu") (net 6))
 (segment (start 132.453553 66.2) (end 148.3 66.2) (width 0.2) (layer "F.Cu") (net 9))
 (segment (start 128.273864 70.379689) (end 132.453553 66.2) (width 0.2) (layer "F.Cu") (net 9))
 (segment (start 138.4 78.5) (end 134.794175 78.5) (width 0.2) (layer "F.Cu") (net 2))
 (segment (start 134.794175 78.5) (end 131.573864 75.279689) (width 0.2) (layer "F.Cu") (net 2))
 (segment (start 167.606372 71.1) (end 151.6 71.1) (width 0.2) (layer "F.Cu") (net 7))
 (segment (start 168.310488 70.395884) (end 167.606372 71.1) (width 0.2) (layer "F.Cu") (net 7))
 (segment (start 175.263501 118.999309) (end 175.263501 78.948897) (width 0.2) (layer "F.Cu") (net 5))
 (segment (start 175.263501 78.948897) (end 171.610488 75.295884) (width 0.2) (layer "F.Cu") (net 5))
 (segment (start 174.512501 119.750309) (end 175.263501 118.999309) (width 0.2) (layer "F.Cu") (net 5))
 (segment (start 133.446403 114.850309) (end 128.606373 119.690339) (width 0.2) (layer "F.Cu") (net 11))
 (segment (start 171.212501 114.850309) (end 133.446403 114.850309) (width 0.2) (layer "F.Cu") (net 11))
 (segment (start 157.4 100.565) (end 156.775 100.565) (width 0.2) (layer "F.Cu") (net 8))
 (segment (start 157.501 101.86572) (end 157.501 100.666) (width 0.2) (layer "F.Cu") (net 8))
 (segment (start 157.501 100.666) (end 157.4 100.565) (width 0.2) (layer "F.Cu") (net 8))
 (segment (start 151.775 100.295) (end 156.505 100.295) (width 0.2) (layer "F.Cu") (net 8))
 (segment (start 147.426 104.706) (end 154.66072 104.706) (width 0.2) (layer "F.Cu") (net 8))
 (segment (start 146.825 104.105) (end 147.426 104.706) (width 0.2) (layer "F.Cu") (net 8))
 (segment (start 156.505 100.295) (end 156.775 100.565) (width 0.2) (layer "F.Cu") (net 8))
 (segment (start 154.66072 104.706) (end 157.501 101.86572) (width 0.2) (layer "F.Cu") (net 8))
 (segment (start 158.9 83.9) (end 159 84) (width 0.2) (layer "F.Cu") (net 4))
 (segment (start 156.2 83.9) (end 158.9 83.9) (width 0.2) (layer "F.Cu") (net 4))
 (segment (start 145.6 78.5) (end 147.1 80) (width 0.2) (layer "F.Cu") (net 1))
 (segment (start 141.5 78.5) (end 145.6 78.5) (width 0.2) (layer "F.Cu") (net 1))
 (segment (start 147.1 80) (end 147.1 80.6) (width 0.2) (layer "F.Cu") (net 1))
 (segment (start 143.699 79.899) (end 143.298 80.3) (width 0.2) (layer "F.Cu") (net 15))
 (segment (start 146.3 80.6) (end 146.3 80.198) (width 0.2) (layer "F.Cu") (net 15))
 (segment (start 143.298 100.282999) (end 145.850001 102.835) (width 0.2) (layer "F.Cu") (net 15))
 (segment (start 143.298 80.3) (end 143.298 100.282999) (width 0.2) (layer "F.Cu") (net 15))
 (segment (start 146.3 80.198) (end 146.001 79.899) (width 0.2) (layer "F.Cu") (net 15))
 (segment (start 146.001 79.899) (end 143.699 79.899) (width 0.2) (layer "F.Cu") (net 15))
 (segment (start 145.850001 102.835) (end 146.825 102.835) (width 0.2) (layer "F.Cu") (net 15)))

